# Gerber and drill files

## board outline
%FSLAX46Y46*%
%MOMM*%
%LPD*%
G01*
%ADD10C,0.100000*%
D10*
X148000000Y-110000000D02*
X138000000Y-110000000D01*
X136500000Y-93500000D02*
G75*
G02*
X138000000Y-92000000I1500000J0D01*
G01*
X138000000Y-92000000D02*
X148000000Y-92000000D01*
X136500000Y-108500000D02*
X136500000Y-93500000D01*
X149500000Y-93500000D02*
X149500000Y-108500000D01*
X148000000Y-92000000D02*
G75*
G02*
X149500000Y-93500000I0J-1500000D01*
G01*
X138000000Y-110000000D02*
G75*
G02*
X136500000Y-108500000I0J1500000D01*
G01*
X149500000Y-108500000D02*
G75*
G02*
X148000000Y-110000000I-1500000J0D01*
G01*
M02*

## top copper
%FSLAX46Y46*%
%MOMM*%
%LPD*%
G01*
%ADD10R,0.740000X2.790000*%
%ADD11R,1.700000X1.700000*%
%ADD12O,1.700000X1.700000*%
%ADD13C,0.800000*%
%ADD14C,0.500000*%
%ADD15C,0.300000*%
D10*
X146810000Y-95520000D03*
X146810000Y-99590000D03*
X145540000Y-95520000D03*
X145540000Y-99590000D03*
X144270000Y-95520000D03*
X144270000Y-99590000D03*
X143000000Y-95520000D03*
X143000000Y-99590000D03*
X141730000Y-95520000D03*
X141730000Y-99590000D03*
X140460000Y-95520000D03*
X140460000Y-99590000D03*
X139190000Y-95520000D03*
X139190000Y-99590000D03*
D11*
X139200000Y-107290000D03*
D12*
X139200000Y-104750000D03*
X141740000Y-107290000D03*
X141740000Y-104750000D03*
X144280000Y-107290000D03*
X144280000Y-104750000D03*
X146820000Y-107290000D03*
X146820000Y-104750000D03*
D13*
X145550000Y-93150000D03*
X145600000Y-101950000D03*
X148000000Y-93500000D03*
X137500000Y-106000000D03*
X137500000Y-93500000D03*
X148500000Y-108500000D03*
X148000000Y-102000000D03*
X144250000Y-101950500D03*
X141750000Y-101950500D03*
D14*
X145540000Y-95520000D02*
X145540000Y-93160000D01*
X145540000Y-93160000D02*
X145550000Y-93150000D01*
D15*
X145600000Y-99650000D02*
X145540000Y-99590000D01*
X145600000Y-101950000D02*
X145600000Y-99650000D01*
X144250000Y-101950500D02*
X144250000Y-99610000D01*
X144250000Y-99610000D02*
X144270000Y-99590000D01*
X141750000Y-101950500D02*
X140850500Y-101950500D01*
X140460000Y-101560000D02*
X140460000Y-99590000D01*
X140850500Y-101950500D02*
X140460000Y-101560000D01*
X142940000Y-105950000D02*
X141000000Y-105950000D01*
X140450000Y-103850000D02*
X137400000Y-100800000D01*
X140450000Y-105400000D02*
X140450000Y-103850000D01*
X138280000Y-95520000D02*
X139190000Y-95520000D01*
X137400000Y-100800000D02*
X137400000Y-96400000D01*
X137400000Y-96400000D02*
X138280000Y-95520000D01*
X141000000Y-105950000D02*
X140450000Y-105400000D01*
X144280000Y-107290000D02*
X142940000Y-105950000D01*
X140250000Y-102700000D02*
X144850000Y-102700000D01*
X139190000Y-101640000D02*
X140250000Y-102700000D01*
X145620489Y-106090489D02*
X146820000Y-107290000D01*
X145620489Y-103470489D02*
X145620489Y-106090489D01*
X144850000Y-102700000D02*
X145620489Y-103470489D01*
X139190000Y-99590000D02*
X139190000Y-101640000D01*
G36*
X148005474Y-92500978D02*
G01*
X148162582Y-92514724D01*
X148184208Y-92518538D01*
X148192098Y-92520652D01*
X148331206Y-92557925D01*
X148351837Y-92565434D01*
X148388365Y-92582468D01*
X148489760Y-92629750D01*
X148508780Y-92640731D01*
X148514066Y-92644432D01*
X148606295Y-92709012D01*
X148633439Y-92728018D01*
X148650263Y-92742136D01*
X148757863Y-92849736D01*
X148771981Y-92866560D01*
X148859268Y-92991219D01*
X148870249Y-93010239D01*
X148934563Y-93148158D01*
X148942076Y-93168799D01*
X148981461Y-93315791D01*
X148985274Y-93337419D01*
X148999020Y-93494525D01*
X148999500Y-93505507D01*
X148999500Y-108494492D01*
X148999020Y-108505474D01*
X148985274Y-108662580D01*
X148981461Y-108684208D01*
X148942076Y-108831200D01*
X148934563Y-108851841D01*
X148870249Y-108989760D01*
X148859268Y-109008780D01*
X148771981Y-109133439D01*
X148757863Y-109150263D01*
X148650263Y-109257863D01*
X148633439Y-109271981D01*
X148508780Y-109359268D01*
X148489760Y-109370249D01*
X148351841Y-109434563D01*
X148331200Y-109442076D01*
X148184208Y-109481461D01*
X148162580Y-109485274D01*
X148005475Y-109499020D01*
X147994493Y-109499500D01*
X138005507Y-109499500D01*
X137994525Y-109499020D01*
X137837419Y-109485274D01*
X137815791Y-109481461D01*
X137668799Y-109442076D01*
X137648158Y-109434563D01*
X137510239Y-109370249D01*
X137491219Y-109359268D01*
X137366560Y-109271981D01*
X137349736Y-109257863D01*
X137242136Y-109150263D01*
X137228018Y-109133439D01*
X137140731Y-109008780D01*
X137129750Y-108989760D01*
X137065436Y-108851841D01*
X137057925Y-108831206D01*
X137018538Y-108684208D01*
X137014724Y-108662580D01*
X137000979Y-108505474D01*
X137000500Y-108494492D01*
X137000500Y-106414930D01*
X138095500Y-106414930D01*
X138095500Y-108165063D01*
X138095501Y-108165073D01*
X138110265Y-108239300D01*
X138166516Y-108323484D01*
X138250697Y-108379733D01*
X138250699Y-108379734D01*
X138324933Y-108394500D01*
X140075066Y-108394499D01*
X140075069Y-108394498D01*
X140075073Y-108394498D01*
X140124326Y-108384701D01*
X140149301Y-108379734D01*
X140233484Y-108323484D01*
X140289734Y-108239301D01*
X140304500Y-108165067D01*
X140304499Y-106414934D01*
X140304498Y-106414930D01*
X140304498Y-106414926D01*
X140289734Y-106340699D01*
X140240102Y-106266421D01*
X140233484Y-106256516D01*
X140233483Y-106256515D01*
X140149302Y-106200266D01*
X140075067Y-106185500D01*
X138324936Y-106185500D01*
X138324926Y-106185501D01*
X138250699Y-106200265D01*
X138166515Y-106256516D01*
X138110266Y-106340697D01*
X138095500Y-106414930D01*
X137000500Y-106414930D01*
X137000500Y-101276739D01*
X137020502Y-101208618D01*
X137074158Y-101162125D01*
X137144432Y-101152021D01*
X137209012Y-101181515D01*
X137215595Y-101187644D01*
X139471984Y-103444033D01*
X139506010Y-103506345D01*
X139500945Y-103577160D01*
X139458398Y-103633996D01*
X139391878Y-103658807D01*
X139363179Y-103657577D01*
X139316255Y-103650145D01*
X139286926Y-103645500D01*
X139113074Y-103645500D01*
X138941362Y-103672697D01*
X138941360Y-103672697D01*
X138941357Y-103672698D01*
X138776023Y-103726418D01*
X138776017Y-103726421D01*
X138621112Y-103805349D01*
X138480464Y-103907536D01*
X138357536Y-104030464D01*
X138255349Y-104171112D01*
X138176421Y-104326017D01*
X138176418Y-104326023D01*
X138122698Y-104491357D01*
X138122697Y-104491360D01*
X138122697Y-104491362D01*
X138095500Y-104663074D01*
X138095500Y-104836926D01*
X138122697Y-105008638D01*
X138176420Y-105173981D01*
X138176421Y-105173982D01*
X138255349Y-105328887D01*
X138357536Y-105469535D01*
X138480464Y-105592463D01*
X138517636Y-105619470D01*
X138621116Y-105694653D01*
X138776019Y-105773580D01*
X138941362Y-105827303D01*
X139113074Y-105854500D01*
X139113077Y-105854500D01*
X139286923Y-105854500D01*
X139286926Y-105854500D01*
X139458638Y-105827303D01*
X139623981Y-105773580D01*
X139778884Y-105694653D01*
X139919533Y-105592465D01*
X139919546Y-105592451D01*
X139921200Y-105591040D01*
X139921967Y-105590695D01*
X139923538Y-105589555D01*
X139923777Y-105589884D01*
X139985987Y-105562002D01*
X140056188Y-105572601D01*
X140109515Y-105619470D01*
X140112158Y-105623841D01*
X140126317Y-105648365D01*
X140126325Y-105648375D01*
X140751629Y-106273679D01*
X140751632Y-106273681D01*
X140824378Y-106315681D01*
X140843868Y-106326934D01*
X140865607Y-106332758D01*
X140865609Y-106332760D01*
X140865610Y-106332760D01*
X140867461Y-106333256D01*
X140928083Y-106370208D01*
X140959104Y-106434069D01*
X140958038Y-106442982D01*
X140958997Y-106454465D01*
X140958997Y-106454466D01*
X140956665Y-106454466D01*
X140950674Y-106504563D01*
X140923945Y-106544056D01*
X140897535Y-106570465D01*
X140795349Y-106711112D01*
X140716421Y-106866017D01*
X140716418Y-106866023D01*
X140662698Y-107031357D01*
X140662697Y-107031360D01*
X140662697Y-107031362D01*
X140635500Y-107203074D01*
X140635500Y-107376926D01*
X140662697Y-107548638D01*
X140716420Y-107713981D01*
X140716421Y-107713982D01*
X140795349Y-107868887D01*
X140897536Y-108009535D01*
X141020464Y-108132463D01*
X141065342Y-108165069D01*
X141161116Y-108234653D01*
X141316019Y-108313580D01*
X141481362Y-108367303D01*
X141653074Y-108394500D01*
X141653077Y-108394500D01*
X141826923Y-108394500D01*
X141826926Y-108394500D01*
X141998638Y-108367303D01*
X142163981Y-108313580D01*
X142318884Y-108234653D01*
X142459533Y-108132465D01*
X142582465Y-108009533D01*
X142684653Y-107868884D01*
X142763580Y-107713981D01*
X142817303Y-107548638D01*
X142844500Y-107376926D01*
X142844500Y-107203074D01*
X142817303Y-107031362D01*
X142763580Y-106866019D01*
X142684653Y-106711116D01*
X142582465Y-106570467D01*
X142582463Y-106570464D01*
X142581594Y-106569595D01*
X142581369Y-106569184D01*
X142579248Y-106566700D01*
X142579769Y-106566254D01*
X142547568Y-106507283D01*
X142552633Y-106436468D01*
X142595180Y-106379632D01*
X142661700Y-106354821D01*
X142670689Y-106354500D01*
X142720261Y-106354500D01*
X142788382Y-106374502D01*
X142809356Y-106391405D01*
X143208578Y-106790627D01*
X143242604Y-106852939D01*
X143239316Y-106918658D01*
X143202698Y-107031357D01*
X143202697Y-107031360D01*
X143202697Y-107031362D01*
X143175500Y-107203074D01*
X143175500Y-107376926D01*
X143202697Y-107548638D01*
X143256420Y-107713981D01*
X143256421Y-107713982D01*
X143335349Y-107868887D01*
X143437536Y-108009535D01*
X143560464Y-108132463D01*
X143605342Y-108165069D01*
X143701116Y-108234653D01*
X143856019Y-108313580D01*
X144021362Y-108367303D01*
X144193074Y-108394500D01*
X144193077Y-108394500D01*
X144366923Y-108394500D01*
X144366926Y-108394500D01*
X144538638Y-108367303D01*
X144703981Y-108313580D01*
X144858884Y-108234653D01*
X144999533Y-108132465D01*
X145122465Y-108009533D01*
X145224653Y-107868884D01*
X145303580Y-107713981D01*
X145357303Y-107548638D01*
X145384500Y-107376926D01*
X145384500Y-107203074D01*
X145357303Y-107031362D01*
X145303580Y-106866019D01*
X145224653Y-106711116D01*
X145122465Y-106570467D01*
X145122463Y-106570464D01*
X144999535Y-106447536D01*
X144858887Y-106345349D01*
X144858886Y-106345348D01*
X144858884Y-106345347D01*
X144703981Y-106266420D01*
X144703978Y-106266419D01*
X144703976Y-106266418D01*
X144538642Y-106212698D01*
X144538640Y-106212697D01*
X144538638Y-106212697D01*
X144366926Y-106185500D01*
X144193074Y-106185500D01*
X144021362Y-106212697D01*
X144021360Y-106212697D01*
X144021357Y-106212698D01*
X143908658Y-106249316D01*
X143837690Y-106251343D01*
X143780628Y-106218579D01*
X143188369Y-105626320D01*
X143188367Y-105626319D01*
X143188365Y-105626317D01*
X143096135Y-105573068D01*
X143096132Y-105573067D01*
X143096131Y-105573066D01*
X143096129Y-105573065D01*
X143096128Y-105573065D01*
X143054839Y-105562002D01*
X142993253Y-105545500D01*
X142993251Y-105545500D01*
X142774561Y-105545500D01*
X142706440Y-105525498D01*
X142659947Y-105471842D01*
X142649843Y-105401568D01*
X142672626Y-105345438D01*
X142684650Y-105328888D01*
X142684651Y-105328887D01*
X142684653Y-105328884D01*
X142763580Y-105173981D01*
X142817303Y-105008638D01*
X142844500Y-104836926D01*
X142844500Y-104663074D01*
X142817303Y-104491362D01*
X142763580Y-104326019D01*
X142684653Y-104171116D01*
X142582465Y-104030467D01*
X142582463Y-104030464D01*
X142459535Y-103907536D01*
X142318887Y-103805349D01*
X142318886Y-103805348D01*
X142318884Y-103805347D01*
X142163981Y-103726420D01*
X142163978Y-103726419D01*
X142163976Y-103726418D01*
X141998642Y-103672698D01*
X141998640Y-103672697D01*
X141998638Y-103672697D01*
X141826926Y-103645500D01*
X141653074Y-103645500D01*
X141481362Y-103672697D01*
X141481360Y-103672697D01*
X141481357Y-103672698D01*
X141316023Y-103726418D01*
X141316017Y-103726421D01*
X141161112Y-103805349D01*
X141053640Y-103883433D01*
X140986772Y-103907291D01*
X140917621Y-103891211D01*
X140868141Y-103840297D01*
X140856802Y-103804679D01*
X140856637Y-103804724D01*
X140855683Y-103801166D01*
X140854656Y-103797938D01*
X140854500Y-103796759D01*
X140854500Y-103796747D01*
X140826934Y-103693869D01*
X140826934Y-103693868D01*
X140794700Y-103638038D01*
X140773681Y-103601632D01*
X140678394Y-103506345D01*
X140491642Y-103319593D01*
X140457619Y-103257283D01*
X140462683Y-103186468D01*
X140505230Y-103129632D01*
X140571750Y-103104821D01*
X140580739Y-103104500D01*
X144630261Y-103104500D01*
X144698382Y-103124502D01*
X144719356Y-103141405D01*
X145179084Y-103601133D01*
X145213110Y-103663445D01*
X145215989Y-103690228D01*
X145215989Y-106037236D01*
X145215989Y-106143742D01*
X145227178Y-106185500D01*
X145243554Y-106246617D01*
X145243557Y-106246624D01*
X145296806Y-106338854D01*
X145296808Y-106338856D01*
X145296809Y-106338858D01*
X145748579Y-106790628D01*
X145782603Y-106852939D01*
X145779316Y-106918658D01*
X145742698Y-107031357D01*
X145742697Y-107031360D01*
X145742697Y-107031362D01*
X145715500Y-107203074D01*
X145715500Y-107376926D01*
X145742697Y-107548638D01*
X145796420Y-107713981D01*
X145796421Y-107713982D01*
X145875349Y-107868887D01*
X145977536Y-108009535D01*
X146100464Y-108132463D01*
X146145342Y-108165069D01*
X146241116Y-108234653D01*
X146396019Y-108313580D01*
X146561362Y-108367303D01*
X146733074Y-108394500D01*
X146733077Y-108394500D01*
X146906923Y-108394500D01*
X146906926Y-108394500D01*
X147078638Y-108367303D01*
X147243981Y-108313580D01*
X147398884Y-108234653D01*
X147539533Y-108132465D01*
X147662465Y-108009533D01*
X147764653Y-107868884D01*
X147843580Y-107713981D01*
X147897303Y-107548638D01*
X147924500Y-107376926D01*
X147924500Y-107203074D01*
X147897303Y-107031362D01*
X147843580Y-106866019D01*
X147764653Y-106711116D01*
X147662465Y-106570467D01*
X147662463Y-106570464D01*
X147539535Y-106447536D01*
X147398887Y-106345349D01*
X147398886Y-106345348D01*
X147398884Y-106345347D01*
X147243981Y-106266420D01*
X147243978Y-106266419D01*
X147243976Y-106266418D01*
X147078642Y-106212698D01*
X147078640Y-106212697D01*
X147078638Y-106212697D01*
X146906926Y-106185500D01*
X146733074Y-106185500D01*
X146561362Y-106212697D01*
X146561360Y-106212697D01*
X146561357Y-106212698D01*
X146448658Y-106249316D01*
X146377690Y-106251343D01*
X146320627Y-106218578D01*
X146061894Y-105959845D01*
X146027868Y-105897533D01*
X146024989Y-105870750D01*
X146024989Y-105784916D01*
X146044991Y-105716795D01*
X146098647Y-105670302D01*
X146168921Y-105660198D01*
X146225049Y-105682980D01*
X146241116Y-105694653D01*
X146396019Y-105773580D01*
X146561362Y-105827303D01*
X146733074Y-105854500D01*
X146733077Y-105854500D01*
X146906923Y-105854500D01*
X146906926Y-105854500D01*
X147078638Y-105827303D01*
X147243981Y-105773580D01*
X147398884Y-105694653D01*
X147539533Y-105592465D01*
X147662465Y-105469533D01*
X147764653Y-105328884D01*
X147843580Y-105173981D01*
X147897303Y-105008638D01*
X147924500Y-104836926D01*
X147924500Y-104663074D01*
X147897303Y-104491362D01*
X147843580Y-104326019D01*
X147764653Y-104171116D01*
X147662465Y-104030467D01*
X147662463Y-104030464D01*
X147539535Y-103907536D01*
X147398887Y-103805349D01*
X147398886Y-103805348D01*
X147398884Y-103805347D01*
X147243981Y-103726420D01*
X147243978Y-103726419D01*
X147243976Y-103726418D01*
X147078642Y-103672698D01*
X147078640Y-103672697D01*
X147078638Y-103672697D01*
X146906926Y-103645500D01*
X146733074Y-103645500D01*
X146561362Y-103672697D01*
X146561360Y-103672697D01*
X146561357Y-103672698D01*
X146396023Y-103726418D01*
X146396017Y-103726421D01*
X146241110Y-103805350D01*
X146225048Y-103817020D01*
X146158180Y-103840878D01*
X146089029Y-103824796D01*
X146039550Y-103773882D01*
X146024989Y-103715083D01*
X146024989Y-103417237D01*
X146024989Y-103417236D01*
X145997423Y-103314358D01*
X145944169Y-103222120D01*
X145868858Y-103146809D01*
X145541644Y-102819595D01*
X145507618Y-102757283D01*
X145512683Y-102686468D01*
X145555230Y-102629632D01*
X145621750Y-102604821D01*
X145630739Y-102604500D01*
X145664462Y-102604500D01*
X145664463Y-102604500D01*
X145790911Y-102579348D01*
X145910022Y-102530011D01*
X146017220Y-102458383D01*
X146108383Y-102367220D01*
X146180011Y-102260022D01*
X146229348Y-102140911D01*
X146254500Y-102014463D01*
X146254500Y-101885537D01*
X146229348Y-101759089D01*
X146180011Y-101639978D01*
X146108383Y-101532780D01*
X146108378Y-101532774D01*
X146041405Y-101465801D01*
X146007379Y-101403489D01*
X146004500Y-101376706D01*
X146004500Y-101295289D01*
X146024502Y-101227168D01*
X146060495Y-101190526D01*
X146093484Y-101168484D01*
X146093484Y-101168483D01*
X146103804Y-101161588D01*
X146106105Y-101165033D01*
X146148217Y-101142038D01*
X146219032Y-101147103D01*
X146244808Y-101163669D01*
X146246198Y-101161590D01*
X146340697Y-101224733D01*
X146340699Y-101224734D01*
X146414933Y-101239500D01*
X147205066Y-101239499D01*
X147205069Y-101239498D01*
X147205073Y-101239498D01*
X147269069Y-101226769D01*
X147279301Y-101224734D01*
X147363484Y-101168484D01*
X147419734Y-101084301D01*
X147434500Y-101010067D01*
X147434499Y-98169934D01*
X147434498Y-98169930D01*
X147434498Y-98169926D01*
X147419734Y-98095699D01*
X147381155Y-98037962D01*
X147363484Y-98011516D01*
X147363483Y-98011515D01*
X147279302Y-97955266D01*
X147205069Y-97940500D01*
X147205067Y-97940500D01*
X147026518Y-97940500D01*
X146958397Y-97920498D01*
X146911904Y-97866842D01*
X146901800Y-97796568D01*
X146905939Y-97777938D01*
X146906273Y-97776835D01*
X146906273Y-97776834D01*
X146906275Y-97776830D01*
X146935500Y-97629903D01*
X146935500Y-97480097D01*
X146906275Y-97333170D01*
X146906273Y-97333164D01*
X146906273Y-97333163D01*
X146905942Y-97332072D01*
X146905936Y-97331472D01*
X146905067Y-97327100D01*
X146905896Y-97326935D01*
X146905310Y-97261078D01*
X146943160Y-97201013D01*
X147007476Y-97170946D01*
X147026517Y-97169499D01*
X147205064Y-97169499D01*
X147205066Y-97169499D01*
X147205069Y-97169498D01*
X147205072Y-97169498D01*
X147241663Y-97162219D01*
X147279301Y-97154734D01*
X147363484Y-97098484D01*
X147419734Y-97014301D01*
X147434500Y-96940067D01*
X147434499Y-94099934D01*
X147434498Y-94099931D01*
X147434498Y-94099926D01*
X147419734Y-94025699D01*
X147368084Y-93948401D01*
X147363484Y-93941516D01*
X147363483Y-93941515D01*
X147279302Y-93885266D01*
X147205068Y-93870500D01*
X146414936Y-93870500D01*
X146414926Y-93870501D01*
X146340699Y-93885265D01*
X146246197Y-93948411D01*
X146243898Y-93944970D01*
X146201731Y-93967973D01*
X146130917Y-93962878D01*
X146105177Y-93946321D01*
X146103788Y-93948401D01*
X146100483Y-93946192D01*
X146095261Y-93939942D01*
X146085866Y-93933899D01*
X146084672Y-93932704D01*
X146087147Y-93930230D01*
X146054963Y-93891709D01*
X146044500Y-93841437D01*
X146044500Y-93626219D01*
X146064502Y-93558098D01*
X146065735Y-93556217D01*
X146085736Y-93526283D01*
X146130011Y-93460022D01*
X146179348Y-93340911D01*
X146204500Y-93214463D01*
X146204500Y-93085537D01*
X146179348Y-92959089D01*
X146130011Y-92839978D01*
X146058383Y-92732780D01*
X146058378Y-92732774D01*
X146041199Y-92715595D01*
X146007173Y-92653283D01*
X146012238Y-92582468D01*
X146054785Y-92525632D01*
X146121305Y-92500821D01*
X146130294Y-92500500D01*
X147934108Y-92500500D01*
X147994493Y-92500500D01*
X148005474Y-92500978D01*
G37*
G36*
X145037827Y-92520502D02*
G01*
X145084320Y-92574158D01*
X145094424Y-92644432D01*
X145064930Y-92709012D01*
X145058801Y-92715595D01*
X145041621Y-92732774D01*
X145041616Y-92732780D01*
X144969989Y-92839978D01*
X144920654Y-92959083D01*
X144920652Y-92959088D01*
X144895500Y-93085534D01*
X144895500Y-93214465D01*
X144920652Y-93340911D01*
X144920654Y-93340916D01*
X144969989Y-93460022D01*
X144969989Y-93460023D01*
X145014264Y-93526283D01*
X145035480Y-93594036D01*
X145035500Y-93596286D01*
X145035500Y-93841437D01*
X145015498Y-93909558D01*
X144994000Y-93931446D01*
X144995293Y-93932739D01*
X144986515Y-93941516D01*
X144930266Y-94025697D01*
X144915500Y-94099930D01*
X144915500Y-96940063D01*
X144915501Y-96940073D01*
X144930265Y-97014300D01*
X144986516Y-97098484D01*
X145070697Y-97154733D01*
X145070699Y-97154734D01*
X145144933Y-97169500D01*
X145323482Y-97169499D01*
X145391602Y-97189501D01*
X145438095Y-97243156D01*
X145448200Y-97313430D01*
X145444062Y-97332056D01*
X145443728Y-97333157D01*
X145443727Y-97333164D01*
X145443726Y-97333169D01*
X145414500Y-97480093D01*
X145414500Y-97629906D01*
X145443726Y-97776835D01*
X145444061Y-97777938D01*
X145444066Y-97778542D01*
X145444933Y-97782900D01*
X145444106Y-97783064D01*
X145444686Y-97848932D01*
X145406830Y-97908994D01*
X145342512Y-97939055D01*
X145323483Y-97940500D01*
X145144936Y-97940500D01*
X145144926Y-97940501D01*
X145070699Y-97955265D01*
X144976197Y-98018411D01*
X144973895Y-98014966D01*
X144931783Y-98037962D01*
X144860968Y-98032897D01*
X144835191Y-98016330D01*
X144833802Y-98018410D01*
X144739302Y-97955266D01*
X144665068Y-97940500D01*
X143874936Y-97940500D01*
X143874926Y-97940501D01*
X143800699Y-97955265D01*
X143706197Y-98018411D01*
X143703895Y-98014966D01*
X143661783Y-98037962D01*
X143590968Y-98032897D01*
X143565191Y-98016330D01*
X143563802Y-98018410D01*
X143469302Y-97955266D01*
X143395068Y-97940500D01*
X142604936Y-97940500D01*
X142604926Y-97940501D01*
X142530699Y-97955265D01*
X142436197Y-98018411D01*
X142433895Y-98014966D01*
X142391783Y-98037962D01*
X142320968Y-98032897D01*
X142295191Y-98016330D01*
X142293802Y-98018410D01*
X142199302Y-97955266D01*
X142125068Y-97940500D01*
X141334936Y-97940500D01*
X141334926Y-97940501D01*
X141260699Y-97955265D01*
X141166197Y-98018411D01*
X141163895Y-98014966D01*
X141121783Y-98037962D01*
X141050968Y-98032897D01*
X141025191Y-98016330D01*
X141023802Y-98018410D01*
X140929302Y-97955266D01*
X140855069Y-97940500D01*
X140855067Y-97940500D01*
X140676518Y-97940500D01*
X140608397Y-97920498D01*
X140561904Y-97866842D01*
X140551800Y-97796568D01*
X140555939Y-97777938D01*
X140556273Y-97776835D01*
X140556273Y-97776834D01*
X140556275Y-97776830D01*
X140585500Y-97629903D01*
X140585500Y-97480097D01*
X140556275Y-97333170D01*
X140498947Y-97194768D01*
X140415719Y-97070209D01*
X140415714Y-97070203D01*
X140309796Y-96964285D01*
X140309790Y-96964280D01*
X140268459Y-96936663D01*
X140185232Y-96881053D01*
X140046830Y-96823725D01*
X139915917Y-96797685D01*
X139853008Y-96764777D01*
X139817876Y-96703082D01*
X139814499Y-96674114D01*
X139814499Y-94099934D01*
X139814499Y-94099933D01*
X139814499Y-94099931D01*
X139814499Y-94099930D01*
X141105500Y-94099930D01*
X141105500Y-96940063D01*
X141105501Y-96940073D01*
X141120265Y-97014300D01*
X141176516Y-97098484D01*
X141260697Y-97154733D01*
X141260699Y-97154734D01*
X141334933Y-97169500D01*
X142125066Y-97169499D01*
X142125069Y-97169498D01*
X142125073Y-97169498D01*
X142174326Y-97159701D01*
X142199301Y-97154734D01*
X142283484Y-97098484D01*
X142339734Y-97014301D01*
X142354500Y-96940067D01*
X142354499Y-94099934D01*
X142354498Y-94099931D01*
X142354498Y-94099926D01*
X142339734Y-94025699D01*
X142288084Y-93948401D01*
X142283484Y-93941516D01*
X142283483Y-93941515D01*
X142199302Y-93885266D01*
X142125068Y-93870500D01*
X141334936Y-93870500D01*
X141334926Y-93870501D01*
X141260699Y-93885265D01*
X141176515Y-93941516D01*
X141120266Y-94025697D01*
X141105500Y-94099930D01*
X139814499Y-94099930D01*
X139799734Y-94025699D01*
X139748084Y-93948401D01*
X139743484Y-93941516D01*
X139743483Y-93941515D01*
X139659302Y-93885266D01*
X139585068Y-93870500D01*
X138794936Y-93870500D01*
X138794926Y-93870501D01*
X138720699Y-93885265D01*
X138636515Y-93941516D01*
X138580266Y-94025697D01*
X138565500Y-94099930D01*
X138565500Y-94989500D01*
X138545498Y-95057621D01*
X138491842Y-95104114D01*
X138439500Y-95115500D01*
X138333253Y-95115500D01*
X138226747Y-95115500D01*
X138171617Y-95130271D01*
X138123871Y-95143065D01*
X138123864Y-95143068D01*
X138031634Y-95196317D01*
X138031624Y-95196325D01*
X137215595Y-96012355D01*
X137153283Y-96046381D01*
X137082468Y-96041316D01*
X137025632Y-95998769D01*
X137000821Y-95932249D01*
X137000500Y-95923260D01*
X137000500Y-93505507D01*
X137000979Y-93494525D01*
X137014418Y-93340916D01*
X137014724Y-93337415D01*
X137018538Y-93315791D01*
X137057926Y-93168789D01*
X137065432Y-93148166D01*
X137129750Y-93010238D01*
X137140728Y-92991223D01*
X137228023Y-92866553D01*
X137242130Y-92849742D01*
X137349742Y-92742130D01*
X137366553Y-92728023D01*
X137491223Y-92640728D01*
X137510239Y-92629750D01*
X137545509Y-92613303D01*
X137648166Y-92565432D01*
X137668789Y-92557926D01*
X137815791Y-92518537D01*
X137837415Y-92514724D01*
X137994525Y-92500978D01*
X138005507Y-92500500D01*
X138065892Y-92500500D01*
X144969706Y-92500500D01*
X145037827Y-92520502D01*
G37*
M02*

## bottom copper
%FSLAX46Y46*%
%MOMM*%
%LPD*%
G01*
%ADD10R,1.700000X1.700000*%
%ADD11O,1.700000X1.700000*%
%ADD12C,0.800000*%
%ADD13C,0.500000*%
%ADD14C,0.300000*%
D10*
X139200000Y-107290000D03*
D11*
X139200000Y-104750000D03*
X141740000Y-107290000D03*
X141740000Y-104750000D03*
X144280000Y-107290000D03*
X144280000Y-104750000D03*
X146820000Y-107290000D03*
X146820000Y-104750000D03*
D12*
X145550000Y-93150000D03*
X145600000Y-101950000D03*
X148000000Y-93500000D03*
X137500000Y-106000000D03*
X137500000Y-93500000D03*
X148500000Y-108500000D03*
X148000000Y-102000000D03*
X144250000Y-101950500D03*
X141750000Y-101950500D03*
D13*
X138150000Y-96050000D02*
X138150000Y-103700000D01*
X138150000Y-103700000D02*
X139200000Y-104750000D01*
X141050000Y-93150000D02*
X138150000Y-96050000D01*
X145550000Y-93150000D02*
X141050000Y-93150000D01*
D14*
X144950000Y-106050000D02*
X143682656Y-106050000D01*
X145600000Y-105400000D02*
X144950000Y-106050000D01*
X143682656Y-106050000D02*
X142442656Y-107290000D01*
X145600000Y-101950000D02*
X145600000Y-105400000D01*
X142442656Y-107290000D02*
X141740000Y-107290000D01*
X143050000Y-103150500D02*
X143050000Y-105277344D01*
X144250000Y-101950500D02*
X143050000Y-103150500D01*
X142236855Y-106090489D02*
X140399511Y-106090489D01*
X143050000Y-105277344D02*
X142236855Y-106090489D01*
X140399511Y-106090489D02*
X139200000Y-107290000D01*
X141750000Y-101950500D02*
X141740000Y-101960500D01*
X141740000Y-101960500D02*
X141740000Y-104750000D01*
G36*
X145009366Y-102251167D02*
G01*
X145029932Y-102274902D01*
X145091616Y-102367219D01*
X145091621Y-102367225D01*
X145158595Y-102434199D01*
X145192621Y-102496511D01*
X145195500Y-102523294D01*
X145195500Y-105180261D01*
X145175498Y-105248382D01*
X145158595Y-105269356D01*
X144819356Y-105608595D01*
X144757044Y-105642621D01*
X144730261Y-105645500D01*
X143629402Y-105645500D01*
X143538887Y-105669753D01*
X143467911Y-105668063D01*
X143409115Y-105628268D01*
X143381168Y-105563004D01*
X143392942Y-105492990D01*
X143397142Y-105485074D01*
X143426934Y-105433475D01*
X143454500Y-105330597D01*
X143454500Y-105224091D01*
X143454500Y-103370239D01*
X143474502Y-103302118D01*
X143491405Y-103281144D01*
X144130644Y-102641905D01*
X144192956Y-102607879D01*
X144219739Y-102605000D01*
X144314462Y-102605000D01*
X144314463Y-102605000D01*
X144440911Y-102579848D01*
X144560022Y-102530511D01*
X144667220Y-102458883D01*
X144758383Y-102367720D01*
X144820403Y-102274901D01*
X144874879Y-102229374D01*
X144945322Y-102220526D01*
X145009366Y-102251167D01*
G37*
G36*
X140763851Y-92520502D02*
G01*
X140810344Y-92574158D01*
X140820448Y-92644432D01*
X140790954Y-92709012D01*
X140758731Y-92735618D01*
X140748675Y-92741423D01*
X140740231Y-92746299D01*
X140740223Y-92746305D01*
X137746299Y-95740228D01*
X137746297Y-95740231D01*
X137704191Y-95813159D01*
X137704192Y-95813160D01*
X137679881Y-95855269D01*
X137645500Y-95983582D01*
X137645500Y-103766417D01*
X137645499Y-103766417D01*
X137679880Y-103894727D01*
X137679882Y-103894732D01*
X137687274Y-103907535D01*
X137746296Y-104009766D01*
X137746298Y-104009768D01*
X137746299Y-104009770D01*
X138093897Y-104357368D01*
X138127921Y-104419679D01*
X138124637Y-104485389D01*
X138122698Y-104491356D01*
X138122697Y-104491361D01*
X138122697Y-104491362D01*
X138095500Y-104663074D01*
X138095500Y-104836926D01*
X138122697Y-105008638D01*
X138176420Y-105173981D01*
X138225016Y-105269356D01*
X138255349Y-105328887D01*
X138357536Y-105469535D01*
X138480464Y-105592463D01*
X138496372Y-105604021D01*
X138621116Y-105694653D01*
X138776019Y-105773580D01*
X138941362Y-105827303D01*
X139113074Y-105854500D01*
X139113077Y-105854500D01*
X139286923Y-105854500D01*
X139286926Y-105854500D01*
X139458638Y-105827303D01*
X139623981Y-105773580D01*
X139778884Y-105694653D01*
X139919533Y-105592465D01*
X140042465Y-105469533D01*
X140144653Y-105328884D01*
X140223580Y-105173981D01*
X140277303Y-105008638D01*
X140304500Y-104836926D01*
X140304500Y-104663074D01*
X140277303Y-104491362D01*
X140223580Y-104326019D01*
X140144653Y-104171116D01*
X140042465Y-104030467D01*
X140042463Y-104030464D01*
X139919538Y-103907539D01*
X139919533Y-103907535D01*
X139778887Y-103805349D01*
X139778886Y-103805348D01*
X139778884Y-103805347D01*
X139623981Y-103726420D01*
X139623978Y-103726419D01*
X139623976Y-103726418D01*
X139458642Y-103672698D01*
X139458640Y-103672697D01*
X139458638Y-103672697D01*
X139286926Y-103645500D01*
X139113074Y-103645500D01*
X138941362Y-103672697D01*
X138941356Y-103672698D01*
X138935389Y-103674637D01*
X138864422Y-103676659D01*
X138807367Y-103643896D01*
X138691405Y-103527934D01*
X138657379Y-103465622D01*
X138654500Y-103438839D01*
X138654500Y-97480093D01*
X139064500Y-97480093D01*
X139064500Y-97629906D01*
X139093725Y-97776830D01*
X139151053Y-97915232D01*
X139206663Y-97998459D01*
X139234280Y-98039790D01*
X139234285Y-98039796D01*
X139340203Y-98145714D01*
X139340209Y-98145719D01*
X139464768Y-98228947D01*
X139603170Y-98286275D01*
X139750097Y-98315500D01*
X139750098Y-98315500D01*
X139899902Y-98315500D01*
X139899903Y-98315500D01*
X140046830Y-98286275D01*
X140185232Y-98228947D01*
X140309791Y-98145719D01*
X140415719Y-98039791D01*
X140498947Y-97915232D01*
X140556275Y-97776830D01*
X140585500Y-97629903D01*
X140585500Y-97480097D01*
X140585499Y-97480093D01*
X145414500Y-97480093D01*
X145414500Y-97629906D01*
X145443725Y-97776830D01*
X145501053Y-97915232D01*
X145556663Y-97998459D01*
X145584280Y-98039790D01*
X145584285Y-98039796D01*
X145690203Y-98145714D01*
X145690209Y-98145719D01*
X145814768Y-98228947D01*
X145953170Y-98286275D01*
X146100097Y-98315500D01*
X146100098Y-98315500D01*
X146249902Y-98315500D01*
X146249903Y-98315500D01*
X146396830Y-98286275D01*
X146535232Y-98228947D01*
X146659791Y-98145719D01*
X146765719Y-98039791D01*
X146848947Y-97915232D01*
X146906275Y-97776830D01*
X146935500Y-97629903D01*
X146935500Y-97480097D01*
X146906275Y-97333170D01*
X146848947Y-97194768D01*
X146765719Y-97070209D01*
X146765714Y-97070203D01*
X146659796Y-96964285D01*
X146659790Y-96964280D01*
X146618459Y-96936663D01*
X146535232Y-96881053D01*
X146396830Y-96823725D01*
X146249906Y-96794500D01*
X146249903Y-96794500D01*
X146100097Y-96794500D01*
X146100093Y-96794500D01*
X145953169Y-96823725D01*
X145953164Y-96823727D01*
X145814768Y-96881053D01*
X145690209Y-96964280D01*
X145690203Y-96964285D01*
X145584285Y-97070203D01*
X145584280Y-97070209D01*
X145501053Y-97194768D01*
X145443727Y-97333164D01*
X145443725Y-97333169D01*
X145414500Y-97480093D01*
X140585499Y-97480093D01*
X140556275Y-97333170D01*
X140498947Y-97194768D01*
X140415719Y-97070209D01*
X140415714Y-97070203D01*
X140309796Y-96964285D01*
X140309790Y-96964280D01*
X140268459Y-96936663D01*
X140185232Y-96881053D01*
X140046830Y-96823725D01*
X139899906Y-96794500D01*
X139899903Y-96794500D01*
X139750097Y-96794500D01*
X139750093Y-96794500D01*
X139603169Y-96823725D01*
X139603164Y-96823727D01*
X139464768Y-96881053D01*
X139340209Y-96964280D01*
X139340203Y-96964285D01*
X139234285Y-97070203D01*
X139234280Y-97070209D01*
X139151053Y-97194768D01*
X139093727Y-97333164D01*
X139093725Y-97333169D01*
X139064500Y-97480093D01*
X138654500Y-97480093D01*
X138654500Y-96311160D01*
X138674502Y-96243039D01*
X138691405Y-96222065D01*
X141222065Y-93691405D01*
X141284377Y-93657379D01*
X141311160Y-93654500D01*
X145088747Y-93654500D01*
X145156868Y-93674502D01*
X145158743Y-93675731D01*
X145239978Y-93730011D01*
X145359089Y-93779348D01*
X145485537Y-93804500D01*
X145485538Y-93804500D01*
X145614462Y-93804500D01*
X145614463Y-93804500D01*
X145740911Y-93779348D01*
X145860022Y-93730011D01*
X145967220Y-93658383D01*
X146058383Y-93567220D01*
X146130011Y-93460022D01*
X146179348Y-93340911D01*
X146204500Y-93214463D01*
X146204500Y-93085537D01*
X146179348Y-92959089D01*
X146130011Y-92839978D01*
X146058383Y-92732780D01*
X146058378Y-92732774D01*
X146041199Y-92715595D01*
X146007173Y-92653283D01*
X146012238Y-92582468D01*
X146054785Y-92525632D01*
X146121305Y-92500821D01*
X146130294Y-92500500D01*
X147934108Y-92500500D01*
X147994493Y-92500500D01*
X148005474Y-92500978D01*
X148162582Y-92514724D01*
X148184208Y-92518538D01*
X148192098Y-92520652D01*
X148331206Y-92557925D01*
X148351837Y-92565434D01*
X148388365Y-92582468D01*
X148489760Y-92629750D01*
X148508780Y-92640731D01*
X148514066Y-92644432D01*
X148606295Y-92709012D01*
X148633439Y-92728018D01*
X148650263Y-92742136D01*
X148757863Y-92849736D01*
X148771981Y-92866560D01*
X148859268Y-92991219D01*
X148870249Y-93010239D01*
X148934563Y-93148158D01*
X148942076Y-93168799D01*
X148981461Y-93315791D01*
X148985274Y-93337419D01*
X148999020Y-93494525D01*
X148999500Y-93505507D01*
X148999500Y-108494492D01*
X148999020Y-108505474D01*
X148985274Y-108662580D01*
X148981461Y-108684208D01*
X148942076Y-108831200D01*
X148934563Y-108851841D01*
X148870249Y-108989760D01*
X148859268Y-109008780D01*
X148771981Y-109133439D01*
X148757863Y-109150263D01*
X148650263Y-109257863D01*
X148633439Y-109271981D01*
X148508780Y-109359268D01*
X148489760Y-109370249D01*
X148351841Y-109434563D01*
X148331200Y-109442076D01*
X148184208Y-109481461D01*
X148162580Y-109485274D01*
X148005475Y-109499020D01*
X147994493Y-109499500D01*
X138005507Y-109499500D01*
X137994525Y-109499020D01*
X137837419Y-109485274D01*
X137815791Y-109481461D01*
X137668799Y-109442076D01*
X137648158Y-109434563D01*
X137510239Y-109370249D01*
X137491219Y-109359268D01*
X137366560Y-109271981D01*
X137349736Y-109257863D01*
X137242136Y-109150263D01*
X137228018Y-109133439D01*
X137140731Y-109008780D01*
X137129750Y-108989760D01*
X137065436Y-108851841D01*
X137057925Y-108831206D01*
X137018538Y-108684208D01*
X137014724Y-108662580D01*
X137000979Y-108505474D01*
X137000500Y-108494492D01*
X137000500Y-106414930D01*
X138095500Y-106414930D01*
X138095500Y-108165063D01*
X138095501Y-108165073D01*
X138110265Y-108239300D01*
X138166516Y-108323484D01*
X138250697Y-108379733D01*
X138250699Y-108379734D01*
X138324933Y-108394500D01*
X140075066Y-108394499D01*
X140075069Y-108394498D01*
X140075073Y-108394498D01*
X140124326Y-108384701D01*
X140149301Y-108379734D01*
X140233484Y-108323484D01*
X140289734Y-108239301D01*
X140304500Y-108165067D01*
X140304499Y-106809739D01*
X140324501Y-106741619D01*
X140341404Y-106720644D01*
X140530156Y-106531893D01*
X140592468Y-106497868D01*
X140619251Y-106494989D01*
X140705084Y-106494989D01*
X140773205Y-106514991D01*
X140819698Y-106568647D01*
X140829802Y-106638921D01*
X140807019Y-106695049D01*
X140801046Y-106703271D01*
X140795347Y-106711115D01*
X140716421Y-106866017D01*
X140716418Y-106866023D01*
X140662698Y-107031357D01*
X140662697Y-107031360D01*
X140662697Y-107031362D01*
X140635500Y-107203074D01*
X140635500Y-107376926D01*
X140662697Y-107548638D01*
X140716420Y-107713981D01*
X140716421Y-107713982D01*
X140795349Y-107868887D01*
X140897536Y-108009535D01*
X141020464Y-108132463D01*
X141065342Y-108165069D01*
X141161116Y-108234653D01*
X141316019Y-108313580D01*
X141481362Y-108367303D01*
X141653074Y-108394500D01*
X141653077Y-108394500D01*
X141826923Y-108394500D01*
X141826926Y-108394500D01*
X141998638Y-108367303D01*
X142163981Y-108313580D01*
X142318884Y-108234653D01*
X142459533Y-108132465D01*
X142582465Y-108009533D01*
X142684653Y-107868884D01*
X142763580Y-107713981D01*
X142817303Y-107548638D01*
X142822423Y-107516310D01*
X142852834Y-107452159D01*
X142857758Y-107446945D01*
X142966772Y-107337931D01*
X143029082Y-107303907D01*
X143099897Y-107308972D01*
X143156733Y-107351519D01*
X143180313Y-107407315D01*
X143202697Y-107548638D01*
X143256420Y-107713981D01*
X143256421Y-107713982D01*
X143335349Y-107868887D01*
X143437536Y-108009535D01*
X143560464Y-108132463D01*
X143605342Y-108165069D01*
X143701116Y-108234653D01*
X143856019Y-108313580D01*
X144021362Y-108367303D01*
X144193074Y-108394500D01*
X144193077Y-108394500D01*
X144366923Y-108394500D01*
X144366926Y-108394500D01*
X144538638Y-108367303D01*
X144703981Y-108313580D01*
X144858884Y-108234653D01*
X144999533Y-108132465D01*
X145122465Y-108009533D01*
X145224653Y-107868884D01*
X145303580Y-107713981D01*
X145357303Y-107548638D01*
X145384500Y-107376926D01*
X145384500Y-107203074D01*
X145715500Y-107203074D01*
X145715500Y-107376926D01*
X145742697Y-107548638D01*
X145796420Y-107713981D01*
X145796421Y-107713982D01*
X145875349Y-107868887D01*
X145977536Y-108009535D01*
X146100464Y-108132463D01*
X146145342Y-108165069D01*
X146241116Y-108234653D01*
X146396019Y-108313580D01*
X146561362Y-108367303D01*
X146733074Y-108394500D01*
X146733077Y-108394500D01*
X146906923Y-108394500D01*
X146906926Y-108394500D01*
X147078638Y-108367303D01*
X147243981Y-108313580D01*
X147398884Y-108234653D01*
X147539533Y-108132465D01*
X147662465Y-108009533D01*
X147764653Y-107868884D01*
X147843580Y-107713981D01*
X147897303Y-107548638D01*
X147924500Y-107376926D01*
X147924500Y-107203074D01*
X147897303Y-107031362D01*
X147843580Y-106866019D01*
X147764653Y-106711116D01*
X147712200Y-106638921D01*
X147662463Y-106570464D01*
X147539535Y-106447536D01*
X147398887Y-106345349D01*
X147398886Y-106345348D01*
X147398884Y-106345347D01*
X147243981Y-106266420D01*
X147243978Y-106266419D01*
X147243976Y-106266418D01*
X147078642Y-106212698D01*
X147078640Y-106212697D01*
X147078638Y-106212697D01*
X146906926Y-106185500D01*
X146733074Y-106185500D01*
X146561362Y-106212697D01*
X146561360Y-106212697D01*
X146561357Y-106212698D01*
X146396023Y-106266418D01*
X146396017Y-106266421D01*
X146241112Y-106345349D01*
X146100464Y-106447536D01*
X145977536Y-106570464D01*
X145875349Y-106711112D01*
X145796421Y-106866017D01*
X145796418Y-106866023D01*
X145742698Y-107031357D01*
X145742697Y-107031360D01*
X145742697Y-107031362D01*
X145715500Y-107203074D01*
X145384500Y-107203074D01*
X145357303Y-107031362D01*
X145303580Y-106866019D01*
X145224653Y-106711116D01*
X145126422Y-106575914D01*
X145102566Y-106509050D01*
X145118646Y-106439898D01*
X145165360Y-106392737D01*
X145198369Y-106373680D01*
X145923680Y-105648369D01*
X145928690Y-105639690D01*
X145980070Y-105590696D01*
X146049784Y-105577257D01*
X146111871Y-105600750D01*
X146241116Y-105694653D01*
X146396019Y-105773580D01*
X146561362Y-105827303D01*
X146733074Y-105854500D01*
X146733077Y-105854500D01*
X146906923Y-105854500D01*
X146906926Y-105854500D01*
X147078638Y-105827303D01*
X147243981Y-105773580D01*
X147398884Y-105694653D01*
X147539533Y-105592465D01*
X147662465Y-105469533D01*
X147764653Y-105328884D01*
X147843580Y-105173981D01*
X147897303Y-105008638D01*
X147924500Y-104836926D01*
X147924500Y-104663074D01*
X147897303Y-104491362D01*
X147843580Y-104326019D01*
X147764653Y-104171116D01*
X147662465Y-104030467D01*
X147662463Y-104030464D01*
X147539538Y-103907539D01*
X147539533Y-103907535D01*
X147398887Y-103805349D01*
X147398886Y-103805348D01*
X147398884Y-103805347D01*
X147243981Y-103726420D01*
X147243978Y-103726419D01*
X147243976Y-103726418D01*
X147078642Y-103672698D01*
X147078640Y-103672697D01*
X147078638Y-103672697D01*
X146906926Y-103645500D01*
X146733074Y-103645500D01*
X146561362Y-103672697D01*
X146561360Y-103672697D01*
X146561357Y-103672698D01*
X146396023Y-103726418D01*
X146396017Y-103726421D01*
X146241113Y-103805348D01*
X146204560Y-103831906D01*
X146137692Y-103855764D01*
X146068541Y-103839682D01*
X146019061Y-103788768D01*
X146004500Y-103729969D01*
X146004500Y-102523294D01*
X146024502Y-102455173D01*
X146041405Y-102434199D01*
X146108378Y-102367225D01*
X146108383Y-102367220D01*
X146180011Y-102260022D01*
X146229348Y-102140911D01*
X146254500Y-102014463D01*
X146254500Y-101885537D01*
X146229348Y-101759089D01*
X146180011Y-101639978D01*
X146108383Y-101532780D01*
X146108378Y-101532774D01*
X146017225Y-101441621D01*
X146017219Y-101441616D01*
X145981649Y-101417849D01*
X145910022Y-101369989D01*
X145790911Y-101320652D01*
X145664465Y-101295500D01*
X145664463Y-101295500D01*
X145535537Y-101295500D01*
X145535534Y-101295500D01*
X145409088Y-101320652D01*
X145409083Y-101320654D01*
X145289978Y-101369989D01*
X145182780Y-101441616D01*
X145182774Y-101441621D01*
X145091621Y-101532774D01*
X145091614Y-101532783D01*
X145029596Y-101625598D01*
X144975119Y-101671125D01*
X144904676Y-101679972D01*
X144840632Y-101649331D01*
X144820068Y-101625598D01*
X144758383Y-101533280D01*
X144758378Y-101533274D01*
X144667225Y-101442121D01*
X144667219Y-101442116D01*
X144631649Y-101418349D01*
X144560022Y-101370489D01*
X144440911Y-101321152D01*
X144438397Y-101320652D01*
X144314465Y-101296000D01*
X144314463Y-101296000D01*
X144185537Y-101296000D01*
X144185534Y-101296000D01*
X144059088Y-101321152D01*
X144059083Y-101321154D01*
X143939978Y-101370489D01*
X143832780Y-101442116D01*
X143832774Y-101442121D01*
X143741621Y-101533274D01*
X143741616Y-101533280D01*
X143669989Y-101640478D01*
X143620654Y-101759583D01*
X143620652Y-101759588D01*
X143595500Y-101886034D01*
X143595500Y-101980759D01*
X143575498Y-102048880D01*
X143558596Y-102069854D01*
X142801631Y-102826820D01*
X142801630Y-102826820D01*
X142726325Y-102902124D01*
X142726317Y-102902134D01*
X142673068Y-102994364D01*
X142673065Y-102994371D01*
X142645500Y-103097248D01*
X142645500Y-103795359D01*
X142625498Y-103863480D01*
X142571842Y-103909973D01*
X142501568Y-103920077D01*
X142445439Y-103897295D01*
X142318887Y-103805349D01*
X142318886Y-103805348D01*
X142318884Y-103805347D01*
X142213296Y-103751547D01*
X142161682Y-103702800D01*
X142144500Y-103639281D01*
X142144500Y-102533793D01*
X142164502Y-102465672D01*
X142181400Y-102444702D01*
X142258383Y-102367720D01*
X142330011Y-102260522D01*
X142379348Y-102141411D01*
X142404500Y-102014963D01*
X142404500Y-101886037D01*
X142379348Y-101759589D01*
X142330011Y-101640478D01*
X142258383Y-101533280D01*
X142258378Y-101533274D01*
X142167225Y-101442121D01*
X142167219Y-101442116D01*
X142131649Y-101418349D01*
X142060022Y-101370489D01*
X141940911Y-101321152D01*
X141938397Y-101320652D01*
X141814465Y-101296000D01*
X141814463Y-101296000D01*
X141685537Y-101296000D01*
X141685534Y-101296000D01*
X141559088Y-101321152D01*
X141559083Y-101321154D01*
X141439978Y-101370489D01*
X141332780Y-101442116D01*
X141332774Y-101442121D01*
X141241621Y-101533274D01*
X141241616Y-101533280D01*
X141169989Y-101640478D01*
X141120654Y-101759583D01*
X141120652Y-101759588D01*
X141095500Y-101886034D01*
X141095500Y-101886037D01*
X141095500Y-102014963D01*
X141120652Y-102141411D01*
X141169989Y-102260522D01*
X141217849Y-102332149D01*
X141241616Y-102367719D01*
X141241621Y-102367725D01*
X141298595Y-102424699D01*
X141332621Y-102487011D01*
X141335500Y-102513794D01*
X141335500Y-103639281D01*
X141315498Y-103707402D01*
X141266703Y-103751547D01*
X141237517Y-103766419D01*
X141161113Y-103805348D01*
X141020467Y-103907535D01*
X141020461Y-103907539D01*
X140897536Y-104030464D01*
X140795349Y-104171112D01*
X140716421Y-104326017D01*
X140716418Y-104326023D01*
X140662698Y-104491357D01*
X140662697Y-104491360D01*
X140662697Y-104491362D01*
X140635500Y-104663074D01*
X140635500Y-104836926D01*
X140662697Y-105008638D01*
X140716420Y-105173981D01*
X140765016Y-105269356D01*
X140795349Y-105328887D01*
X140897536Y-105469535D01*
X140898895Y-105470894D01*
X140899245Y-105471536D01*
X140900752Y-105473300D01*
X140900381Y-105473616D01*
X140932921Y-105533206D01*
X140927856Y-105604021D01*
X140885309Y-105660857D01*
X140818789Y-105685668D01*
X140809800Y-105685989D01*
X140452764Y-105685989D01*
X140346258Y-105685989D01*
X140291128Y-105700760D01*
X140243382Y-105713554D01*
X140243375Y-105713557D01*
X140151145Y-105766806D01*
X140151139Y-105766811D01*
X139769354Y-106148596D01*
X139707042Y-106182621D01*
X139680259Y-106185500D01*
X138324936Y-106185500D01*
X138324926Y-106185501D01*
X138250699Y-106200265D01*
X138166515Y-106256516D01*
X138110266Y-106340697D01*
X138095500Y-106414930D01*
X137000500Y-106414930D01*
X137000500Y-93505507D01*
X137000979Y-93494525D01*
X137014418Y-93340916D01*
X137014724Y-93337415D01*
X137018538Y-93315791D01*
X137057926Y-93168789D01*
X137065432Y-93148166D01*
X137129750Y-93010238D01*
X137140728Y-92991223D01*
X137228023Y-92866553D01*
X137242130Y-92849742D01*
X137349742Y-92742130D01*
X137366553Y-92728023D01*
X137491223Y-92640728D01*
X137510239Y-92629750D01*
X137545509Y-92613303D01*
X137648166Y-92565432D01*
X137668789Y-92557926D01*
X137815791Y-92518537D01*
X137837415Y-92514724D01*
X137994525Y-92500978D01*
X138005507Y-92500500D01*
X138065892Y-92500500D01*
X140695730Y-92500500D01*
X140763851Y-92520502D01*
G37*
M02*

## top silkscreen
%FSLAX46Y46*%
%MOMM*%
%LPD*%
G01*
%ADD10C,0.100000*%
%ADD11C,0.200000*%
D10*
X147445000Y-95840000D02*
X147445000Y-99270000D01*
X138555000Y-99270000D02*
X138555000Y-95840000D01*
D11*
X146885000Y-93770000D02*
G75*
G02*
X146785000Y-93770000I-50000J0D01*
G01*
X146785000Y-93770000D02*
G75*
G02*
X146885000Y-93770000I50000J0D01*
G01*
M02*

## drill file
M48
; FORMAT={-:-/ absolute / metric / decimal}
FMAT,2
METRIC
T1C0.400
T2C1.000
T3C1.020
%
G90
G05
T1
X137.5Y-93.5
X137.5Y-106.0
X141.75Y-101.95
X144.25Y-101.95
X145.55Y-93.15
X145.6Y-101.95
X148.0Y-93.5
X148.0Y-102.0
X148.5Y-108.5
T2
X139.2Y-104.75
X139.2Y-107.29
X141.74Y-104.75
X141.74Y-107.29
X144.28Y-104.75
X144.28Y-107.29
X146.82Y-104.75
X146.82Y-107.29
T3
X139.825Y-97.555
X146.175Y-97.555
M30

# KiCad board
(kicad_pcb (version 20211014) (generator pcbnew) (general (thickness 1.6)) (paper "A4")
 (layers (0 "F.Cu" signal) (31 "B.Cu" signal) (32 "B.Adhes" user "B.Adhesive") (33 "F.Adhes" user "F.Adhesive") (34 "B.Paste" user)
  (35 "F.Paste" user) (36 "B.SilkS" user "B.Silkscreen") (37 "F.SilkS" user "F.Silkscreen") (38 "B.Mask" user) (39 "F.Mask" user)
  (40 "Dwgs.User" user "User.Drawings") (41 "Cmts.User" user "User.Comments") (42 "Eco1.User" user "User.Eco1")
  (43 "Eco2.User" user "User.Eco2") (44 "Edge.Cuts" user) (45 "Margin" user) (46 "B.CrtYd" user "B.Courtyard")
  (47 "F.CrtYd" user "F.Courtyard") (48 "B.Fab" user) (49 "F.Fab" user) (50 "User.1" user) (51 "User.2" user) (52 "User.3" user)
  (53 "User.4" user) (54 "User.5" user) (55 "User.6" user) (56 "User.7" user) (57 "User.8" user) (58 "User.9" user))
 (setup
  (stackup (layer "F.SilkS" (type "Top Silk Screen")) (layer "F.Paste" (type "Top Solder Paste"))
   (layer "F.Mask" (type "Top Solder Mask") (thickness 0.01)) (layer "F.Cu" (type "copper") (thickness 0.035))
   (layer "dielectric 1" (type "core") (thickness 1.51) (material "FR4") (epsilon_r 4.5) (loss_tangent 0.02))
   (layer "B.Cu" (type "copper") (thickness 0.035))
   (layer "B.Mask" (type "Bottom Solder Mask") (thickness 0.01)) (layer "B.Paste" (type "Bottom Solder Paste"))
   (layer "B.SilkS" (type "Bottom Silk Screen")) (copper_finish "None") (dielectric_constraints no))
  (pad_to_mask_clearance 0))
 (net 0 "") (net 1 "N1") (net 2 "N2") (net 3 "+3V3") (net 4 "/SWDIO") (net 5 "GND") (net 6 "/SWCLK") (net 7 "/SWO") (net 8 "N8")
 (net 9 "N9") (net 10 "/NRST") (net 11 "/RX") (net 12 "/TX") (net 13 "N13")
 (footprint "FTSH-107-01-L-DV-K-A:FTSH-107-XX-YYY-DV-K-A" (layer "F.Cu") (at 143 97.555 180)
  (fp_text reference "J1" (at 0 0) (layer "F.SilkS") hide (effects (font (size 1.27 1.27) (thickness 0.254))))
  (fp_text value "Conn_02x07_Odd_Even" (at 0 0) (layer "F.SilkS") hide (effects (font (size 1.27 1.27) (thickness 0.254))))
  (fp_line (start -4.445 1.715) (end -4.445 -1.715) (layer "F.SilkS") (width 0.1))
  (fp_line (start 4.445 -1.715) (end 4.445 1.715) (layer "F.SilkS") (width 0.1))
  (fp_circle (center -3.835 3.785) (end -3.835 3.835) (layer "F.SilkS") (width 0.2) (fill none))
  (pad "" np_thru_hole circle locked (at -3.175 0 180) (size 1.02 1.02) (drill 1.02) (layers *.Cu *.Mask))
  (pad "" np_thru_hole circle locked (at 3.175 0 180) (size 1.02 1.02) (drill 1.02) (layers *.Cu *.Mask))
  (pad "1" smd rect locked (at -3.81 2.035 180) (size 0.74 2.79) (layers "F.Cu" "F.Paste" "F.Mask") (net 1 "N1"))
  (pad "2" smd rect locked (at -3.81 -2.035 180) (size 0.74 2.79) (layers "F.Cu" "F.Paste" "F.Mask") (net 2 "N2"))
  (pad "3" smd rect locked (at -2.54 2.035 180) (size 0.74 2.79) (layers "F.Cu" "F.Paste" "F.Mask") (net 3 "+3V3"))
  (pad "4" smd rect locked (at -2.54 -2.035 180) (size 0.74 2.79) (layers "F.Cu" "F.Paste" "F.Mask") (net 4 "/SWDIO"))
  (pad "5" smd rect locked (at -1.27 2.035 180) (size 0.74 2.79) (layers "F.Cu" "F.Paste" "F.Mask") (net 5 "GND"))
  (pad "6" smd rect locked (at -1.27 -2.035 180) (size 0.74 2.79) (layers "F.Cu" "F.Paste" "F.Mask") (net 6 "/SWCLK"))
  (pad "7" smd rect locked (at 0 2.035 180) (size 0.74 2.79) (layers "F.Cu" "F.Paste" "F.Mask") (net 5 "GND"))
  (pad "8" smd rect locked (at 0 -2.035 180) (size 0.74 2.79) (layers "F.Cu" "F.Paste" "F.Mask") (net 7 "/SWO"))
  (pad "9" smd rect locked (at 1.27 2.035 180) (size 0.74 2.79) (layers "F.Cu" "F.Paste" "F.Mask") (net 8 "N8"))
  (pad "10" smd rect locked (at 1.27 -2.035 180) (size 0.74 2.79) (layers "F.Cu" "F.Paste" "F.Mask") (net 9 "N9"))
  (pad "11" smd rect locked (at 2.54 2.035 180) (size 0.74 2.79) (layers "F.Cu" "F.Paste" "F.Mask") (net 5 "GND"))
  (pad "12" smd rect locked (at 2.54 -2.035 180) (size 0.74 2.79) (layers "F.Cu" "F.Paste" "F.Mask") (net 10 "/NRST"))
  (pad "13" smd rect locked (at 3.81 2.035 180) (size 0.74 2.79) (layers "F.Cu" "F.Paste" "F.Mask") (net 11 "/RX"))
  (pad "14" smd rect locked (at 3.81 -2.035 180) (size 0.74 2.79) (layers "F.Cu" "F.Paste" "F.Mask") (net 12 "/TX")))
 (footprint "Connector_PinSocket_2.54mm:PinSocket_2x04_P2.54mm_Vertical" (layer "B.Cu") (at 139.2 107.29 -90)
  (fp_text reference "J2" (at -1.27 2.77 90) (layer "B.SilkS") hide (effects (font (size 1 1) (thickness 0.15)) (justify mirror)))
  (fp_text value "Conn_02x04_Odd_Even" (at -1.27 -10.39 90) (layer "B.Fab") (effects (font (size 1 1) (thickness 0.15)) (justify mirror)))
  (pad "1" thru_hole rect locked (at 0 0 270) (size 1.7 1.7) (drill 1) (layers *.Cu *.Mask) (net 6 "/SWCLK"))
  (pad "2" thru_hole oval locked (at -2.54 0 270) (size 1.7 1.7) (drill 1) (layers *.Cu *.Mask) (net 3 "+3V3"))
  (pad "3" thru_hole oval locked (at 0 -2.54 270) (size 1.7 1.7) (drill 1) (layers *.Cu *.Mask) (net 4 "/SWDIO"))
  (pad "4" thru_hole oval locked (at -2.54 -2.54 270) (size 1.7 1.7) (drill 1) (layers *.Cu *.Mask) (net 10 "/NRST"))
  (pad "5" thru_hole oval locked (at 0 -5.08 270) (size 1.7 1.7) (drill 1) (layers *.Cu *.Mask) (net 11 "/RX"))
  (pad "6" thru_hole oval locked (at -2.54 -5.08 270) (size 1.7 1.7) (drill 1) (layers *.Cu *.Mask) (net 5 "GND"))
  (pad "7" thru_hole oval locked (at 0 -7.62 270) (size 1.7 1.7) (drill 1) (layers *.Cu *.Mask) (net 12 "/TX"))
  (pad "8" thru_hole oval locked (at -2.54 -7.62 270) (size 1.7 1.7) (drill 1) (layers *.Cu *.Mask) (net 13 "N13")))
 (gr_line (start 148 110) (end 138 110) (layer "Edge.Cuts") (width 0.1))
 (gr_arc (start 136.5 93.5) (mid 136.93934 92.43934) (end 138 92) (layer "Edge.Cuts") (width 0.1))
 (gr_line (start 138 92) (end 148 92) (layer "Edge.Cuts") (width 0.1))
 (gr_line (start 136.5 108.5) (end 136.5 93.5) (layer "Edge.Cuts") (width 0.1))
 (gr_line (start 149.5 93.5) (end 149.5 108.5) (layer "Edge.Cuts") (width 0.1))
 (gr_arc (start 148 92) (mid 149.06066 92.43934) (end 149.5 93.5) (layer "Edge.Cuts") (width 0.1))
 (gr_arc (start 138 110) (mid 136.93934 109.56066) (end 136.5 108.5) (layer "Edge.Cuts") (width 0.1))
 (gr_arc (start 149.5 108.5) (mid 149.06066 109.56066) (end 148 110) (layer "Edge.Cuts") (width 0.1))
 (segment (start 145.54 95.52) (end 145.54 93.16) (width 0.5) (layer "F.Cu") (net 3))
 (segment (start 145.54 93.16) (end 145.55 93.15) (width 0.5) (layer "F.Cu") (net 3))
 (via (at 145.55 93.15) (size 0.8) (drill 0.4) (layers "F.Cu" "B.Cu") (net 3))
 (segment (start 138.15 96.05) (end 138.15 103.7) (width 0.5) (layer "B.Cu") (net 3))
 (segment (start 138.15 103.7) (end 139.2 104.75) (width 0.5) (layer "B.Cu") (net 3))
 (segment (start 141.05 93.15) (end 138.15 96.05) (width 0.5) (layer "B.Cu") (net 3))
 (segment (start 145.55 93.15) (end 141.05 93.15) (width 0.5) (layer "B.Cu") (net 3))
 (segment (start 145.6 99.65) (end 145.54 99.59) (width 0.3) (layer "F.Cu") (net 4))
 (segment (start 145.6 101.95) (end 145.6 99.65) (width 0.3) (layer "F.Cu") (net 4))
 (via (at 145.6 101.95) (size 0.8) (drill 0.4) (layers "F.Cu" "B.Cu") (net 4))
 (segment (start 144.95 106.05) (end 143.682656 106.05) (width 0.3) (layer "B.Cu") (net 4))
 (segment (start 145.6 105.4) (end 144.95 106.05) (width 0.3) (layer "B.Cu") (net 4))
 (segment (start 143.682656 106.05) (end 142.442656 107.29) (width 0.3) (layer "B.Cu") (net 4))
 (segment (start 145.6 101.95) (end 145.6 105.4) (width 0.3) (layer "B.Cu") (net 4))
 (segment (start 142.442656 107.29) (end 141.74 107.29) (width 0.3) (layer "B.Cu") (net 4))
 (via (at 148 93.5) (size 0.8) (drill 0.4) (layers "F.Cu" "B.Cu") (free) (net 5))
 (via (at 137.5 106) (size 0.8) (drill 0.4) (layers "F.Cu" "B.Cu") (free) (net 5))
 (via (at 137.5 93.5) (size 0.8) (drill 0.4) (layers "F.Cu" "B.Cu") (free) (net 5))
 (via (at 148.5 108.5) (size 0.8) (drill 0.4) (layers "F.Cu" "B.Cu") (free) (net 5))
 (via (at 148 102) (size 0.8) (drill 0.4) (layers "F.Cu" "B.Cu") (free) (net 5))
 (segment (start 144.25 101.9505) (end 144.25 99.61) (width 0.3) (layer "F.Cu") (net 6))
 (segment (start 144.25 99.61) (end 144.27 99.59) (width 0.3) (layer "F.Cu") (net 6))
 (via (at 144.25 101.9505) (size 0.8) (drill 0.4) (layers "F.Cu" "B.Cu") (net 6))
 (segment (start 143.05 103.1505) (end 143.05 105.277344) (width 0.3) (layer "B.Cu") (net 6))
 (segment (start 144.25 101.9505) (end 143.05 103.1505) (width 0.3) (layer "B.Cu") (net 6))
 (segment (start 142.236855 106.090489) (end 140.399511 106.090489) (width 0.3) (layer "B.Cu") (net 6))
 (segment (start 143.05 105.277344) (end 142.236855 106.090489) (width 0.3) (layer "B.Cu") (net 6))
 (segment (start 140.399511 106.090489) (end 139.2 107.29) (width 0.3) (layer "B.Cu") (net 6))
 (segment (start 141.75 101.9505) (end 140.8505 101.9505) (width 0.3) (layer "F.Cu") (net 10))
 (segment (start 140.46 101.56) (end 140.46 99.59) (width 0.3) (layer "F.Cu") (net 10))
 (segment (start 140.8505 101.9505) (end 140.46 101.56) (width 0.3) (layer "F.Cu") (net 10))
 (via (at 141.75 101.9505) (size 0.8) (drill 0.4) (layers "F.Cu" "B.Cu") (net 10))
 (segment (start 141.75 101.9505) (end 141.74 101.9605) (width 0.3) (layer "B.Cu") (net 10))
 (segment (start 141.74 101.9605) (end 141.74 104.75) (width 0.3) (layer "B.Cu") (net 10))
 (segment (start 142.94 105.95) (end 141 105.95) (width 0.3) (layer "F.Cu") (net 11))
 (segment (start 140.45 103.85) (end 137.4 100.8) (width 0.3) (layer "F.Cu") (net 11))
 (segment (start 140.45 105.4) (end 140.45 103.85) (width 0.3) (layer "F.Cu") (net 11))
 (segment (start 138.28 95.52) (end 139.19 95.52) (width 0.3) (layer "F.Cu") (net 11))
 (segment (start 137.4 100.8) (end 137.4 96.4) (width 0.3) (layer "F.Cu") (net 11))
 (segment (start 137.4 96.4) (end 138.28 95.52) (width 0.3) (layer "F.Cu") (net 11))
 (segment (start 141 105.95) (end 140.45 105.4) (width 0.3) (layer "F.Cu") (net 11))
 (segment (start 144.28 107.29) (end 142.94 105.95) (width 0.3) (layer "F.Cu") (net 11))
 (segment (start 140.25 102.7) (end 144.85 102.7) (width 0.3) (layer "F.Cu") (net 12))
 (segment (start 139.19 101.64) (end 140.25 102.7) (width 0.3) (layer "F.Cu") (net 12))
 (segment (start 145.620489 106.090489) (end 146.82 107.29) (width 0.3) (layer "F.Cu") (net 12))
 (segment (start 145.620489 103.470489) (end 145.620489 106.090489) (width 0.3) (layer "F.Cu") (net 12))
 (segment (start 144.85 102.7) (end 145.620489 103.470489) (width 0.3) (layer "F.Cu") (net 12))
 (segment (start 139.19 99.59) (end 139.19 101.64) (width 0.3) (layer "F.Cu") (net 12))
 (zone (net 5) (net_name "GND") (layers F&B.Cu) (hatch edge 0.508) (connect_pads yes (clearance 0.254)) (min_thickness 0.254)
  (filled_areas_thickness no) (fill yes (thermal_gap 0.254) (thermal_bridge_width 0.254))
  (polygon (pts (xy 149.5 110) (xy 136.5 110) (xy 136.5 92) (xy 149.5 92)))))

